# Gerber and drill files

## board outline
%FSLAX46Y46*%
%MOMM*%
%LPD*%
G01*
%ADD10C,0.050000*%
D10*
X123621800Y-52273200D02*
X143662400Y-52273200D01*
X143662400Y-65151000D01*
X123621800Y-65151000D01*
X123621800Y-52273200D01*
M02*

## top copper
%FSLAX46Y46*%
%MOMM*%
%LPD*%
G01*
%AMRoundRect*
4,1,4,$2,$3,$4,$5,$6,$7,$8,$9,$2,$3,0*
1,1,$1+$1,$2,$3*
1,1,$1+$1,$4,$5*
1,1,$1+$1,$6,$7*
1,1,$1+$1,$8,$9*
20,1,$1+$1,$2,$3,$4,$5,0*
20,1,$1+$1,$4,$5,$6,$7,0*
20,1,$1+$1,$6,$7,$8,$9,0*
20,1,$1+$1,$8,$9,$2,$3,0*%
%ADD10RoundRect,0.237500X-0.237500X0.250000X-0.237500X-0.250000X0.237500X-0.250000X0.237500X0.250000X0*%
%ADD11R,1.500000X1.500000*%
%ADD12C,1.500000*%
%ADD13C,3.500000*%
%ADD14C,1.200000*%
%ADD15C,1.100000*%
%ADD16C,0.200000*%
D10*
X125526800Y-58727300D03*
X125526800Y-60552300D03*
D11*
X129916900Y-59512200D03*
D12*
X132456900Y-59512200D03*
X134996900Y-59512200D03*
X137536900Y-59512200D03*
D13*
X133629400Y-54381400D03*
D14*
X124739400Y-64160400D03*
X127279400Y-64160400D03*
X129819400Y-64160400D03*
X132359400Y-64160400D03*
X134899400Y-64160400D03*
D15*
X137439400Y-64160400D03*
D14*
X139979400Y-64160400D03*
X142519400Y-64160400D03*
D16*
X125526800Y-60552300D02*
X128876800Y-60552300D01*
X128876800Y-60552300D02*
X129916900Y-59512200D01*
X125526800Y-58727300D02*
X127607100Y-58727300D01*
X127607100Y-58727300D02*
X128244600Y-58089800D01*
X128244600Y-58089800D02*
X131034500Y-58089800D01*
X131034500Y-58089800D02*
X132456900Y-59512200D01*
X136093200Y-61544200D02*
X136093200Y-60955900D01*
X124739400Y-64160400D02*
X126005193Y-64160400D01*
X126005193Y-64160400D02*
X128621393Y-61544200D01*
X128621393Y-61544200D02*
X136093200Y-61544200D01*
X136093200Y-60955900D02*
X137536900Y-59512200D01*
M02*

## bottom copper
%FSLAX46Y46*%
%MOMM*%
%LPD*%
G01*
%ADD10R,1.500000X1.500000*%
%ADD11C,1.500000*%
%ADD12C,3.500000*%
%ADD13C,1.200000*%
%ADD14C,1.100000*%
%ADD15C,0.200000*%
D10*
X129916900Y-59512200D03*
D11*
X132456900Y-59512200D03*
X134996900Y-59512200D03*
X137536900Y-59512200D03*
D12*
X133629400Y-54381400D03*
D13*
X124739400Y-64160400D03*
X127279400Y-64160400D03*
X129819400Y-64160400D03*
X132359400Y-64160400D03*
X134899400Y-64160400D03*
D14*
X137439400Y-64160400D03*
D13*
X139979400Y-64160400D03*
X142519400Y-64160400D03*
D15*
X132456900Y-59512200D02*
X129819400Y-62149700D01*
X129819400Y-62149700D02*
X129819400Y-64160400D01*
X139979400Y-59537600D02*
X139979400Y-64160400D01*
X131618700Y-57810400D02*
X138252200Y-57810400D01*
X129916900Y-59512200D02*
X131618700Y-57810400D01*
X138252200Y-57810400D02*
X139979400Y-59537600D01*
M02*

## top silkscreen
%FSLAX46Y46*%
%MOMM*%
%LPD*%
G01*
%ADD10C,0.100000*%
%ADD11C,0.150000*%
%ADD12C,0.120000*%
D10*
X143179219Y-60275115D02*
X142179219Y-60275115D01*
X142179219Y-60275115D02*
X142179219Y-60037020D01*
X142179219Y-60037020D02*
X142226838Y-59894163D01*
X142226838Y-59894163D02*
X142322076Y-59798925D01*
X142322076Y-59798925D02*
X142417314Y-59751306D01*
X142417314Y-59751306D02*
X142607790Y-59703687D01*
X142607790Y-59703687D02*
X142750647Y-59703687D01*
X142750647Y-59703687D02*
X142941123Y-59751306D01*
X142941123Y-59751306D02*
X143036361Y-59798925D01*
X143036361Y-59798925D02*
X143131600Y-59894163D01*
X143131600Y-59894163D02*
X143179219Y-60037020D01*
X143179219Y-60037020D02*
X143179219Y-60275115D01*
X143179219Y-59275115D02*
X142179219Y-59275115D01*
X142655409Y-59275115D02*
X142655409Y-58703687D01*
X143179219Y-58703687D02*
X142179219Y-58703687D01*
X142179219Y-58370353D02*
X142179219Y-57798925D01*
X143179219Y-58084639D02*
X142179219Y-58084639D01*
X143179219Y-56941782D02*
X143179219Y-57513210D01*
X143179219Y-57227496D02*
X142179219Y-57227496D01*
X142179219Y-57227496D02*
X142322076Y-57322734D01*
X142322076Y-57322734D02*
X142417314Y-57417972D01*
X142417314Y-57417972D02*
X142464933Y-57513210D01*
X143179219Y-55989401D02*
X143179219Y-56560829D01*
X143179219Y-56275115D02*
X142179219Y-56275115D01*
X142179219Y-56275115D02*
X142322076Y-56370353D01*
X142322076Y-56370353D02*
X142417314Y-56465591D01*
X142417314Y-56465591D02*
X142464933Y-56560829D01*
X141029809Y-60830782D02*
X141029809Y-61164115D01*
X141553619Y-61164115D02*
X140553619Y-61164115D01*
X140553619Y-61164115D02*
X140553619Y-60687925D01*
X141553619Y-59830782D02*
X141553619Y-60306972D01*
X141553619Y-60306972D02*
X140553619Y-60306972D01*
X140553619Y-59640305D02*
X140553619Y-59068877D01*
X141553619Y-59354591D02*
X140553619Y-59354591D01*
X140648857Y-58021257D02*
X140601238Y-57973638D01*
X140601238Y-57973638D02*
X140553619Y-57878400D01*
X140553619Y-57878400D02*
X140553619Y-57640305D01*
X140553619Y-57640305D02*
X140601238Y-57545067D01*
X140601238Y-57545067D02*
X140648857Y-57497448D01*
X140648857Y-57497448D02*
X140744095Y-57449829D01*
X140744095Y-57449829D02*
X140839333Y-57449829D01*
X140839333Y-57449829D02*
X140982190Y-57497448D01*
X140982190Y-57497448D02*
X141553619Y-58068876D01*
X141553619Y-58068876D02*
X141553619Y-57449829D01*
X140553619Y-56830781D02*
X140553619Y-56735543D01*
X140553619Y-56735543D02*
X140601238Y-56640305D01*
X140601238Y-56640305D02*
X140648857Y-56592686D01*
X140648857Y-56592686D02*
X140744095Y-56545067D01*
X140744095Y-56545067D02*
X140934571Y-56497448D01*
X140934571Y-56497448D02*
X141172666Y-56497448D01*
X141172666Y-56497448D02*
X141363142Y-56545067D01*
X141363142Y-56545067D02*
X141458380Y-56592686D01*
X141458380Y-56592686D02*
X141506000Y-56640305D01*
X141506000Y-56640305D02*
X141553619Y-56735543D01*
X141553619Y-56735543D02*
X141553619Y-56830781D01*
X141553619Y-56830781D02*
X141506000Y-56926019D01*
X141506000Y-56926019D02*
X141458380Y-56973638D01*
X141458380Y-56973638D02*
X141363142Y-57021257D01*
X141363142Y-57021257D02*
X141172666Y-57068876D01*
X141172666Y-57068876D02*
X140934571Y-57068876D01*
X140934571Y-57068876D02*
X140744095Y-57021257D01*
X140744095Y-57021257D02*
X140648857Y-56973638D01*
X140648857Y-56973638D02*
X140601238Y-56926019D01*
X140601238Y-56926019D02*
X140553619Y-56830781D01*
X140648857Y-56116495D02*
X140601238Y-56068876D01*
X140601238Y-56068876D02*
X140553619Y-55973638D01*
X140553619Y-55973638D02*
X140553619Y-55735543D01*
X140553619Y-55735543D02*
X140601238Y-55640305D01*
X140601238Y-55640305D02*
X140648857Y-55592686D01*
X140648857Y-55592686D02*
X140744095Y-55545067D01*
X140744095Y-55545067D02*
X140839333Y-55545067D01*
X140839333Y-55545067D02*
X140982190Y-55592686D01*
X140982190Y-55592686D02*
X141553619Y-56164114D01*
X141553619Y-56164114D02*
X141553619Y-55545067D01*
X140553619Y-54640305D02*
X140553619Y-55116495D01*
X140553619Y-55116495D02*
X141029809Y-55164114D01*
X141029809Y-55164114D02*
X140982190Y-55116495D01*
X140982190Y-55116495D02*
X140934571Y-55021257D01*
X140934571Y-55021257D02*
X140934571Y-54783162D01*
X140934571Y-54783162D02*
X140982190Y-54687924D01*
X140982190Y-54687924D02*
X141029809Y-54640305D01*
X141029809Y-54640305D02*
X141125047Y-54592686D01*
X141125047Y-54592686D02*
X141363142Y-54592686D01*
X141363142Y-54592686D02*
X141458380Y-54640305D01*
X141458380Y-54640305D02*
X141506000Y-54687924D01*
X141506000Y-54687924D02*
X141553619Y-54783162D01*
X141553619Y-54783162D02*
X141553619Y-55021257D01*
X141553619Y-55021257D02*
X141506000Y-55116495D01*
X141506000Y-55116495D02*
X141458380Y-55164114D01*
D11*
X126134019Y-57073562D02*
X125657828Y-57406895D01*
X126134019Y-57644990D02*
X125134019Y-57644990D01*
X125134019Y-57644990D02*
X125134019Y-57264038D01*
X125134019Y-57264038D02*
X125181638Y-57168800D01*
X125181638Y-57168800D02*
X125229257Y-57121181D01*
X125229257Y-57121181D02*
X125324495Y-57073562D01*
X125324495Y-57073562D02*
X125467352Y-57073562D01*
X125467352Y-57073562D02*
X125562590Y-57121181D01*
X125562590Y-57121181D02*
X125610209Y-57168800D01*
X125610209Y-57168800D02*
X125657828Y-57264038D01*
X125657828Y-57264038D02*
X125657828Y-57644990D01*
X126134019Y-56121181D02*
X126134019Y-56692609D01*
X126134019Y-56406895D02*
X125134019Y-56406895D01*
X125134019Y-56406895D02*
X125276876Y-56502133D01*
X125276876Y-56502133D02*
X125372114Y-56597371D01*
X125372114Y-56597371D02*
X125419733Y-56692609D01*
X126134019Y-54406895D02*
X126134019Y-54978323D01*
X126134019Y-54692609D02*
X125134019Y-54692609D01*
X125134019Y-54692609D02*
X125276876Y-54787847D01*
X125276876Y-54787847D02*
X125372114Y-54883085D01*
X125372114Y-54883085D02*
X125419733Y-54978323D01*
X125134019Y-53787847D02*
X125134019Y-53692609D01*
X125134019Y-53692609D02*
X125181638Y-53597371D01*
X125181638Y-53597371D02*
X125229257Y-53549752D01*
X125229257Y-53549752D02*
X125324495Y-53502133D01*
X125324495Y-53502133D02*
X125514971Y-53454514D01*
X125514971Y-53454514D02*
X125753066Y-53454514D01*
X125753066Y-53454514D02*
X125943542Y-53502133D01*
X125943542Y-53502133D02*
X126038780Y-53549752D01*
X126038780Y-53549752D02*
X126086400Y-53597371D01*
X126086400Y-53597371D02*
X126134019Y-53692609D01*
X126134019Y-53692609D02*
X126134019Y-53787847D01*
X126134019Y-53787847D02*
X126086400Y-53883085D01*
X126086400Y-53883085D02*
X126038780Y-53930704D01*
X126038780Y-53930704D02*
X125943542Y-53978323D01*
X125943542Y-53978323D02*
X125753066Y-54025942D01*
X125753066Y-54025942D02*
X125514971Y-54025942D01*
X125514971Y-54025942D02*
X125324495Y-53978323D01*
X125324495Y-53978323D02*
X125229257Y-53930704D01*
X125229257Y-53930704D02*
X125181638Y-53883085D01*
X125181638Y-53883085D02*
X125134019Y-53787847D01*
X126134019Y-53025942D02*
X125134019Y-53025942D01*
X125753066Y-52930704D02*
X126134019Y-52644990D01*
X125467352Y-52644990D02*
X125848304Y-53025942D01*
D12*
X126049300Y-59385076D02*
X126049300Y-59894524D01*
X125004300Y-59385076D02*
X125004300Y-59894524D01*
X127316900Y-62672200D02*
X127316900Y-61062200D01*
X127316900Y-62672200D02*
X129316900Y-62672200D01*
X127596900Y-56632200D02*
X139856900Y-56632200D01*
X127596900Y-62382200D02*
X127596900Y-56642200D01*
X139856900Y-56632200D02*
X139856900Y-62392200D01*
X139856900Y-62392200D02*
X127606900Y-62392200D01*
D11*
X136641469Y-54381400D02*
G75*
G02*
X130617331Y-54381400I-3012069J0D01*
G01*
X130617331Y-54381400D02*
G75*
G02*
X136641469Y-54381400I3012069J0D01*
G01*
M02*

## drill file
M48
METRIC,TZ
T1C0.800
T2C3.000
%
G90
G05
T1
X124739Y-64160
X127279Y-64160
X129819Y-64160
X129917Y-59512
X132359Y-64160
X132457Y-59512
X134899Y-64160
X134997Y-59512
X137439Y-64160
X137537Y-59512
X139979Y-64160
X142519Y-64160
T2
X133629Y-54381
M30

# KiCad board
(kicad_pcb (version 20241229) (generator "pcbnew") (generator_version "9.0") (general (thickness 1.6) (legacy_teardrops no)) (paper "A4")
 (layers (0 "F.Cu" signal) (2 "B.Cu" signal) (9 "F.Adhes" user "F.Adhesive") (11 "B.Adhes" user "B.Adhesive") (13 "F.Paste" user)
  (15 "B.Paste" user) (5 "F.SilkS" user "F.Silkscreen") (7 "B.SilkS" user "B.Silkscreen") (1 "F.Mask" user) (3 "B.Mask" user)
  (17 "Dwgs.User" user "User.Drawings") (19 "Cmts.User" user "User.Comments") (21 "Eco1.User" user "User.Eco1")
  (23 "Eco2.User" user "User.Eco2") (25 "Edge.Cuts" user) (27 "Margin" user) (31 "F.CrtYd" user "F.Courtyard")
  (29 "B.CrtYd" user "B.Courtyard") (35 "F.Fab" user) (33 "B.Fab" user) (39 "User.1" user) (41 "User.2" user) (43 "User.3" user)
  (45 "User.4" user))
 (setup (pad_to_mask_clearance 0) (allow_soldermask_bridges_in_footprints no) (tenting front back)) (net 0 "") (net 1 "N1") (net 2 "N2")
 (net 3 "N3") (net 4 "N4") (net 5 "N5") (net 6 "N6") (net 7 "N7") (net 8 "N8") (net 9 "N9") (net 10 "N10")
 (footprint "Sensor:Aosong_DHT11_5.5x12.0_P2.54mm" (layer "F.Cu") (at 129.9169 59.5122 90)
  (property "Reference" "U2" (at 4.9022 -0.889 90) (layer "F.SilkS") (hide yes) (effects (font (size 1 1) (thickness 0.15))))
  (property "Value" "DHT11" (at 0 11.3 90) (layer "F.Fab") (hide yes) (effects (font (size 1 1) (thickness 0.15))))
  (fp_line (start -3.16 -2.6) (end -1.55 -2.6) (stroke (width 0.12) (type solid)) (layer "F.SilkS"))
  (fp_line (start -3.16 -2.6) (end -3.16 -0.6) (stroke (width 0.12) (type solid)) (layer "F.SilkS"))
  (fp_line (start 2.88 -2.32) (end 2.88 9.94) (stroke (width 0.12) (type solid)) (layer "F.SilkS"))
  (fp_line (start -2.87 -2.32) (end 2.87 -2.32) (stroke (width 0.12) (type solid)) (layer "F.SilkS"))
  (fp_line (start 2.88 9.94) (end -2.88 9.94) (stroke (width 0.12) (type solid)) (layer "F.SilkS"))
  (fp_line (start -2.88 9.94) (end -2.88 -2.31) (stroke (width 0.12) (type solid)) (layer "F.SilkS"))
  (pad "1" thru_hole rect (at 0 0 90) (size 1.5 1.5) (drill 0.8) (layers "*.Cu" "*.Mask") (remove_unused_layers no) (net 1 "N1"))
  (pad "2" thru_hole circle (at 0 2.54 90) (size 1.5 1.5) (drill 0.8) (layers "*.Cu" "*.Mask") (remove_unused_layers no) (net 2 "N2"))
  (pad "3" thru_hole circle (at 0 5.08 90) (size 1.5 1.5) (drill 0.8) (layers "*.Cu" "*.Mask") (remove_unused_layers no) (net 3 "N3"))
  (pad "4" thru_hole circle (at 0 7.62 90) (size 1.5 1.5) (drill 0.8) (layers "*.Cu" "*.Mask") (remove_unused_layers no) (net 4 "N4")))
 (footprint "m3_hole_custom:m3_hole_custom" (layer "F.Cu") (at 133.6294 54.3814)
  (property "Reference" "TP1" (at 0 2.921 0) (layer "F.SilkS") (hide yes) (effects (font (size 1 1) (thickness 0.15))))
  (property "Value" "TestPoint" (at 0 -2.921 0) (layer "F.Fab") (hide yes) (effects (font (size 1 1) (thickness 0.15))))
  (fp_circle (center 0 0) (end 2.8575 0.9525) (stroke (width 0.15) (type solid)) (fill no) (layer "F.SilkS"))
  (pad "1" thru_hole circle (at 0 0) (size 3.5 3.5) (drill 3) (layers "*.Cu" "*.Mask") (remove_unused_layers no) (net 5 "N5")))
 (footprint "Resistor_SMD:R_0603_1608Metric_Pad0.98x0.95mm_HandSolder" (layer "F.Cu") (at 125.5268 59.6398 -90)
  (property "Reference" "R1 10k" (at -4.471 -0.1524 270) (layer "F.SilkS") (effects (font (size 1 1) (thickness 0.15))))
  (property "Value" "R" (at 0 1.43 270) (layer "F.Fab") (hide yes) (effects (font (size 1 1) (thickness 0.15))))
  (fp_line (start -0.254724 0.5225) (end 0.254724 0.5225) (stroke (width 0.12) (type solid)) (layer "F.SilkS"))
  (fp_line (start -0.254724 -0.5225) (end 0.254724 -0.5225) (stroke (width 0.12) (type solid)) (layer "F.SilkS"))
  (pad "1" smd roundrect (at -0.9125 0 270) (size 0.975 0.95) (layers "F.Cu" "F.Mask" "F.Paste") (roundrect_rratio 0.25) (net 2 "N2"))
  (pad "2" smd roundrect (at 0.9125 0 270) (size 0.975 0.95) (layers "F.Cu" "F.Mask" "F.Paste") (roundrect_rratio 0.25) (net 1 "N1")))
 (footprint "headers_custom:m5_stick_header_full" (layer "F.Cu") (at 133.6294 64.1604)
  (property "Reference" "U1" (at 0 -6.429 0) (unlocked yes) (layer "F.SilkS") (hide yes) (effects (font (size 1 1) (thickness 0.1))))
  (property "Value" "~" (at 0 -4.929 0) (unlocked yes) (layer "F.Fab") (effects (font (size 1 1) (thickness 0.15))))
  (pad "1" thru_hole circle (at -8.89 0) (size 1.2 1.2) (drill 0.8) (layers "*.Cu" "*.Mask") (remove_unused_layers no) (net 4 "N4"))
  (pad "2" thru_hole circle (at -6.35 0) (size 1.2 1.2) (drill 0.8) (layers "*.Cu" "*.Mask") (remove_unused_layers no) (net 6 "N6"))
  (pad "3" thru_hole circle (at -3.81 0) (size 1.2 1.2) (drill 0.8) (layers "*.Cu" "*.Mask") (remove_unused_layers no) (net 2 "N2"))
  (pad "4" thru_hole circle (at -1.27 0) (size 1.2 1.2) (drill 0.8) (layers "*.Cu" "*.Mask") (remove_unused_layers no) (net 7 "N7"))
  (pad "5" thru_hole circle (at 1.27 0) (size 1.2 1.2) (drill 0.8) (layers "*.Cu" "*.Mask") (remove_unused_layers no) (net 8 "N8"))
  (pad "6" thru_hole circle (at 3.81 0) (size 1.1 1.1) (drill 0.8) (layers "*.Cu" "*.Mask") (remove_unused_layers no) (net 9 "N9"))
  (pad "7" thru_hole circle (at 6.35 0) (size 1.2 1.2) (drill 0.8) (layers "*.Cu" "*.Mask") (remove_unused_layers no) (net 1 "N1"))
  (pad "8" thru_hole circle (at 8.89 0) (size 1.2 1.2) (drill 0.8) (layers "*.Cu" "*.Mask") (remove_unused_layers no) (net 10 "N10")))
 (gr_rect (start 123.6218 52.2732) (end 143.6624 65.151) (stroke (width 0.05) (type default)) (fill no) (layer "Edge.Cuts"))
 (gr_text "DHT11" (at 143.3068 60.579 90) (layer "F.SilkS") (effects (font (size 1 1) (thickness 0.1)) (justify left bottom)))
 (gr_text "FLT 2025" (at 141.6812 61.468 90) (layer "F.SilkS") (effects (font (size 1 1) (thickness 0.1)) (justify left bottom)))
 (segment (start 128.2446 58.0898) (end 131.0345 58.0898) (width 0.2) (layer "F.Cu") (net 2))
 (segment (start 127.6071 58.7273) (end 128.2446 58.0898) (width 0.2) (layer "F.Cu") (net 2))
 (segment (start 131.0345 58.0898) (end 132.4569 59.5122) (width 0.2) (layer "F.Cu") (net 2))
 (segment (start 125.5268 58.7273) (end 127.6071 58.7273) (width 0.2) (layer "F.Cu") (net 2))
 (segment (start 132.4569 59.5122) (end 129.8194 62.1497) (width 0.2) (layer "B.Cu") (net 2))
 (segment (start 129.8194 62.1497) (end 129.8194 64.1604) (width 0.2) (layer "B.Cu") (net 2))
 (segment (start 125.5268 60.5523) (end 128.8768 60.5523) (width 0.2) (layer "F.Cu") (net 1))
 (segment (start 128.8768 60.5523) (end 129.9169 59.5122) (width 0.2) (layer "F.Cu") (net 1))
 (segment (start 139.9794 59.5376) (end 139.9794 64.1604) (width 0.2) (layer "B.Cu") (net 1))
 (segment (start 131.6187 57.8104) (end 138.2522 57.8104) (width 0.2) (layer "B.Cu") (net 1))
 (segment (start 129.9169 59.5122) (end 131.6187 57.8104) (width 0.2) (layer "B.Cu") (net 1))
 (segment (start 138.2522 57.8104) (end 139.9794 59.5376) (width 0.2) (layer "B.Cu") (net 1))
 (segment (start 136.0932 61.5442) (end 136.0932 60.9559) (width 0.2) (layer "F.Cu") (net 4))
 (segment (start 124.7394 64.1604) (end 126.005193 64.1604) (width 0.2) (layer "F.Cu") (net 4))
 (segment (start 126.005193 64.1604) (end 128.621393 61.5442) (width 0.2) (layer "F.Cu") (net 4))
 (segment (start 128.621393 61.5442) (end 136.0932 61.5442) (width 0.2) (layer "F.Cu") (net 4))
 (segment (start 136.0932 60.9559) (end 137.5369 59.5122) (width 0.2) (layer "F.Cu") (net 4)))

